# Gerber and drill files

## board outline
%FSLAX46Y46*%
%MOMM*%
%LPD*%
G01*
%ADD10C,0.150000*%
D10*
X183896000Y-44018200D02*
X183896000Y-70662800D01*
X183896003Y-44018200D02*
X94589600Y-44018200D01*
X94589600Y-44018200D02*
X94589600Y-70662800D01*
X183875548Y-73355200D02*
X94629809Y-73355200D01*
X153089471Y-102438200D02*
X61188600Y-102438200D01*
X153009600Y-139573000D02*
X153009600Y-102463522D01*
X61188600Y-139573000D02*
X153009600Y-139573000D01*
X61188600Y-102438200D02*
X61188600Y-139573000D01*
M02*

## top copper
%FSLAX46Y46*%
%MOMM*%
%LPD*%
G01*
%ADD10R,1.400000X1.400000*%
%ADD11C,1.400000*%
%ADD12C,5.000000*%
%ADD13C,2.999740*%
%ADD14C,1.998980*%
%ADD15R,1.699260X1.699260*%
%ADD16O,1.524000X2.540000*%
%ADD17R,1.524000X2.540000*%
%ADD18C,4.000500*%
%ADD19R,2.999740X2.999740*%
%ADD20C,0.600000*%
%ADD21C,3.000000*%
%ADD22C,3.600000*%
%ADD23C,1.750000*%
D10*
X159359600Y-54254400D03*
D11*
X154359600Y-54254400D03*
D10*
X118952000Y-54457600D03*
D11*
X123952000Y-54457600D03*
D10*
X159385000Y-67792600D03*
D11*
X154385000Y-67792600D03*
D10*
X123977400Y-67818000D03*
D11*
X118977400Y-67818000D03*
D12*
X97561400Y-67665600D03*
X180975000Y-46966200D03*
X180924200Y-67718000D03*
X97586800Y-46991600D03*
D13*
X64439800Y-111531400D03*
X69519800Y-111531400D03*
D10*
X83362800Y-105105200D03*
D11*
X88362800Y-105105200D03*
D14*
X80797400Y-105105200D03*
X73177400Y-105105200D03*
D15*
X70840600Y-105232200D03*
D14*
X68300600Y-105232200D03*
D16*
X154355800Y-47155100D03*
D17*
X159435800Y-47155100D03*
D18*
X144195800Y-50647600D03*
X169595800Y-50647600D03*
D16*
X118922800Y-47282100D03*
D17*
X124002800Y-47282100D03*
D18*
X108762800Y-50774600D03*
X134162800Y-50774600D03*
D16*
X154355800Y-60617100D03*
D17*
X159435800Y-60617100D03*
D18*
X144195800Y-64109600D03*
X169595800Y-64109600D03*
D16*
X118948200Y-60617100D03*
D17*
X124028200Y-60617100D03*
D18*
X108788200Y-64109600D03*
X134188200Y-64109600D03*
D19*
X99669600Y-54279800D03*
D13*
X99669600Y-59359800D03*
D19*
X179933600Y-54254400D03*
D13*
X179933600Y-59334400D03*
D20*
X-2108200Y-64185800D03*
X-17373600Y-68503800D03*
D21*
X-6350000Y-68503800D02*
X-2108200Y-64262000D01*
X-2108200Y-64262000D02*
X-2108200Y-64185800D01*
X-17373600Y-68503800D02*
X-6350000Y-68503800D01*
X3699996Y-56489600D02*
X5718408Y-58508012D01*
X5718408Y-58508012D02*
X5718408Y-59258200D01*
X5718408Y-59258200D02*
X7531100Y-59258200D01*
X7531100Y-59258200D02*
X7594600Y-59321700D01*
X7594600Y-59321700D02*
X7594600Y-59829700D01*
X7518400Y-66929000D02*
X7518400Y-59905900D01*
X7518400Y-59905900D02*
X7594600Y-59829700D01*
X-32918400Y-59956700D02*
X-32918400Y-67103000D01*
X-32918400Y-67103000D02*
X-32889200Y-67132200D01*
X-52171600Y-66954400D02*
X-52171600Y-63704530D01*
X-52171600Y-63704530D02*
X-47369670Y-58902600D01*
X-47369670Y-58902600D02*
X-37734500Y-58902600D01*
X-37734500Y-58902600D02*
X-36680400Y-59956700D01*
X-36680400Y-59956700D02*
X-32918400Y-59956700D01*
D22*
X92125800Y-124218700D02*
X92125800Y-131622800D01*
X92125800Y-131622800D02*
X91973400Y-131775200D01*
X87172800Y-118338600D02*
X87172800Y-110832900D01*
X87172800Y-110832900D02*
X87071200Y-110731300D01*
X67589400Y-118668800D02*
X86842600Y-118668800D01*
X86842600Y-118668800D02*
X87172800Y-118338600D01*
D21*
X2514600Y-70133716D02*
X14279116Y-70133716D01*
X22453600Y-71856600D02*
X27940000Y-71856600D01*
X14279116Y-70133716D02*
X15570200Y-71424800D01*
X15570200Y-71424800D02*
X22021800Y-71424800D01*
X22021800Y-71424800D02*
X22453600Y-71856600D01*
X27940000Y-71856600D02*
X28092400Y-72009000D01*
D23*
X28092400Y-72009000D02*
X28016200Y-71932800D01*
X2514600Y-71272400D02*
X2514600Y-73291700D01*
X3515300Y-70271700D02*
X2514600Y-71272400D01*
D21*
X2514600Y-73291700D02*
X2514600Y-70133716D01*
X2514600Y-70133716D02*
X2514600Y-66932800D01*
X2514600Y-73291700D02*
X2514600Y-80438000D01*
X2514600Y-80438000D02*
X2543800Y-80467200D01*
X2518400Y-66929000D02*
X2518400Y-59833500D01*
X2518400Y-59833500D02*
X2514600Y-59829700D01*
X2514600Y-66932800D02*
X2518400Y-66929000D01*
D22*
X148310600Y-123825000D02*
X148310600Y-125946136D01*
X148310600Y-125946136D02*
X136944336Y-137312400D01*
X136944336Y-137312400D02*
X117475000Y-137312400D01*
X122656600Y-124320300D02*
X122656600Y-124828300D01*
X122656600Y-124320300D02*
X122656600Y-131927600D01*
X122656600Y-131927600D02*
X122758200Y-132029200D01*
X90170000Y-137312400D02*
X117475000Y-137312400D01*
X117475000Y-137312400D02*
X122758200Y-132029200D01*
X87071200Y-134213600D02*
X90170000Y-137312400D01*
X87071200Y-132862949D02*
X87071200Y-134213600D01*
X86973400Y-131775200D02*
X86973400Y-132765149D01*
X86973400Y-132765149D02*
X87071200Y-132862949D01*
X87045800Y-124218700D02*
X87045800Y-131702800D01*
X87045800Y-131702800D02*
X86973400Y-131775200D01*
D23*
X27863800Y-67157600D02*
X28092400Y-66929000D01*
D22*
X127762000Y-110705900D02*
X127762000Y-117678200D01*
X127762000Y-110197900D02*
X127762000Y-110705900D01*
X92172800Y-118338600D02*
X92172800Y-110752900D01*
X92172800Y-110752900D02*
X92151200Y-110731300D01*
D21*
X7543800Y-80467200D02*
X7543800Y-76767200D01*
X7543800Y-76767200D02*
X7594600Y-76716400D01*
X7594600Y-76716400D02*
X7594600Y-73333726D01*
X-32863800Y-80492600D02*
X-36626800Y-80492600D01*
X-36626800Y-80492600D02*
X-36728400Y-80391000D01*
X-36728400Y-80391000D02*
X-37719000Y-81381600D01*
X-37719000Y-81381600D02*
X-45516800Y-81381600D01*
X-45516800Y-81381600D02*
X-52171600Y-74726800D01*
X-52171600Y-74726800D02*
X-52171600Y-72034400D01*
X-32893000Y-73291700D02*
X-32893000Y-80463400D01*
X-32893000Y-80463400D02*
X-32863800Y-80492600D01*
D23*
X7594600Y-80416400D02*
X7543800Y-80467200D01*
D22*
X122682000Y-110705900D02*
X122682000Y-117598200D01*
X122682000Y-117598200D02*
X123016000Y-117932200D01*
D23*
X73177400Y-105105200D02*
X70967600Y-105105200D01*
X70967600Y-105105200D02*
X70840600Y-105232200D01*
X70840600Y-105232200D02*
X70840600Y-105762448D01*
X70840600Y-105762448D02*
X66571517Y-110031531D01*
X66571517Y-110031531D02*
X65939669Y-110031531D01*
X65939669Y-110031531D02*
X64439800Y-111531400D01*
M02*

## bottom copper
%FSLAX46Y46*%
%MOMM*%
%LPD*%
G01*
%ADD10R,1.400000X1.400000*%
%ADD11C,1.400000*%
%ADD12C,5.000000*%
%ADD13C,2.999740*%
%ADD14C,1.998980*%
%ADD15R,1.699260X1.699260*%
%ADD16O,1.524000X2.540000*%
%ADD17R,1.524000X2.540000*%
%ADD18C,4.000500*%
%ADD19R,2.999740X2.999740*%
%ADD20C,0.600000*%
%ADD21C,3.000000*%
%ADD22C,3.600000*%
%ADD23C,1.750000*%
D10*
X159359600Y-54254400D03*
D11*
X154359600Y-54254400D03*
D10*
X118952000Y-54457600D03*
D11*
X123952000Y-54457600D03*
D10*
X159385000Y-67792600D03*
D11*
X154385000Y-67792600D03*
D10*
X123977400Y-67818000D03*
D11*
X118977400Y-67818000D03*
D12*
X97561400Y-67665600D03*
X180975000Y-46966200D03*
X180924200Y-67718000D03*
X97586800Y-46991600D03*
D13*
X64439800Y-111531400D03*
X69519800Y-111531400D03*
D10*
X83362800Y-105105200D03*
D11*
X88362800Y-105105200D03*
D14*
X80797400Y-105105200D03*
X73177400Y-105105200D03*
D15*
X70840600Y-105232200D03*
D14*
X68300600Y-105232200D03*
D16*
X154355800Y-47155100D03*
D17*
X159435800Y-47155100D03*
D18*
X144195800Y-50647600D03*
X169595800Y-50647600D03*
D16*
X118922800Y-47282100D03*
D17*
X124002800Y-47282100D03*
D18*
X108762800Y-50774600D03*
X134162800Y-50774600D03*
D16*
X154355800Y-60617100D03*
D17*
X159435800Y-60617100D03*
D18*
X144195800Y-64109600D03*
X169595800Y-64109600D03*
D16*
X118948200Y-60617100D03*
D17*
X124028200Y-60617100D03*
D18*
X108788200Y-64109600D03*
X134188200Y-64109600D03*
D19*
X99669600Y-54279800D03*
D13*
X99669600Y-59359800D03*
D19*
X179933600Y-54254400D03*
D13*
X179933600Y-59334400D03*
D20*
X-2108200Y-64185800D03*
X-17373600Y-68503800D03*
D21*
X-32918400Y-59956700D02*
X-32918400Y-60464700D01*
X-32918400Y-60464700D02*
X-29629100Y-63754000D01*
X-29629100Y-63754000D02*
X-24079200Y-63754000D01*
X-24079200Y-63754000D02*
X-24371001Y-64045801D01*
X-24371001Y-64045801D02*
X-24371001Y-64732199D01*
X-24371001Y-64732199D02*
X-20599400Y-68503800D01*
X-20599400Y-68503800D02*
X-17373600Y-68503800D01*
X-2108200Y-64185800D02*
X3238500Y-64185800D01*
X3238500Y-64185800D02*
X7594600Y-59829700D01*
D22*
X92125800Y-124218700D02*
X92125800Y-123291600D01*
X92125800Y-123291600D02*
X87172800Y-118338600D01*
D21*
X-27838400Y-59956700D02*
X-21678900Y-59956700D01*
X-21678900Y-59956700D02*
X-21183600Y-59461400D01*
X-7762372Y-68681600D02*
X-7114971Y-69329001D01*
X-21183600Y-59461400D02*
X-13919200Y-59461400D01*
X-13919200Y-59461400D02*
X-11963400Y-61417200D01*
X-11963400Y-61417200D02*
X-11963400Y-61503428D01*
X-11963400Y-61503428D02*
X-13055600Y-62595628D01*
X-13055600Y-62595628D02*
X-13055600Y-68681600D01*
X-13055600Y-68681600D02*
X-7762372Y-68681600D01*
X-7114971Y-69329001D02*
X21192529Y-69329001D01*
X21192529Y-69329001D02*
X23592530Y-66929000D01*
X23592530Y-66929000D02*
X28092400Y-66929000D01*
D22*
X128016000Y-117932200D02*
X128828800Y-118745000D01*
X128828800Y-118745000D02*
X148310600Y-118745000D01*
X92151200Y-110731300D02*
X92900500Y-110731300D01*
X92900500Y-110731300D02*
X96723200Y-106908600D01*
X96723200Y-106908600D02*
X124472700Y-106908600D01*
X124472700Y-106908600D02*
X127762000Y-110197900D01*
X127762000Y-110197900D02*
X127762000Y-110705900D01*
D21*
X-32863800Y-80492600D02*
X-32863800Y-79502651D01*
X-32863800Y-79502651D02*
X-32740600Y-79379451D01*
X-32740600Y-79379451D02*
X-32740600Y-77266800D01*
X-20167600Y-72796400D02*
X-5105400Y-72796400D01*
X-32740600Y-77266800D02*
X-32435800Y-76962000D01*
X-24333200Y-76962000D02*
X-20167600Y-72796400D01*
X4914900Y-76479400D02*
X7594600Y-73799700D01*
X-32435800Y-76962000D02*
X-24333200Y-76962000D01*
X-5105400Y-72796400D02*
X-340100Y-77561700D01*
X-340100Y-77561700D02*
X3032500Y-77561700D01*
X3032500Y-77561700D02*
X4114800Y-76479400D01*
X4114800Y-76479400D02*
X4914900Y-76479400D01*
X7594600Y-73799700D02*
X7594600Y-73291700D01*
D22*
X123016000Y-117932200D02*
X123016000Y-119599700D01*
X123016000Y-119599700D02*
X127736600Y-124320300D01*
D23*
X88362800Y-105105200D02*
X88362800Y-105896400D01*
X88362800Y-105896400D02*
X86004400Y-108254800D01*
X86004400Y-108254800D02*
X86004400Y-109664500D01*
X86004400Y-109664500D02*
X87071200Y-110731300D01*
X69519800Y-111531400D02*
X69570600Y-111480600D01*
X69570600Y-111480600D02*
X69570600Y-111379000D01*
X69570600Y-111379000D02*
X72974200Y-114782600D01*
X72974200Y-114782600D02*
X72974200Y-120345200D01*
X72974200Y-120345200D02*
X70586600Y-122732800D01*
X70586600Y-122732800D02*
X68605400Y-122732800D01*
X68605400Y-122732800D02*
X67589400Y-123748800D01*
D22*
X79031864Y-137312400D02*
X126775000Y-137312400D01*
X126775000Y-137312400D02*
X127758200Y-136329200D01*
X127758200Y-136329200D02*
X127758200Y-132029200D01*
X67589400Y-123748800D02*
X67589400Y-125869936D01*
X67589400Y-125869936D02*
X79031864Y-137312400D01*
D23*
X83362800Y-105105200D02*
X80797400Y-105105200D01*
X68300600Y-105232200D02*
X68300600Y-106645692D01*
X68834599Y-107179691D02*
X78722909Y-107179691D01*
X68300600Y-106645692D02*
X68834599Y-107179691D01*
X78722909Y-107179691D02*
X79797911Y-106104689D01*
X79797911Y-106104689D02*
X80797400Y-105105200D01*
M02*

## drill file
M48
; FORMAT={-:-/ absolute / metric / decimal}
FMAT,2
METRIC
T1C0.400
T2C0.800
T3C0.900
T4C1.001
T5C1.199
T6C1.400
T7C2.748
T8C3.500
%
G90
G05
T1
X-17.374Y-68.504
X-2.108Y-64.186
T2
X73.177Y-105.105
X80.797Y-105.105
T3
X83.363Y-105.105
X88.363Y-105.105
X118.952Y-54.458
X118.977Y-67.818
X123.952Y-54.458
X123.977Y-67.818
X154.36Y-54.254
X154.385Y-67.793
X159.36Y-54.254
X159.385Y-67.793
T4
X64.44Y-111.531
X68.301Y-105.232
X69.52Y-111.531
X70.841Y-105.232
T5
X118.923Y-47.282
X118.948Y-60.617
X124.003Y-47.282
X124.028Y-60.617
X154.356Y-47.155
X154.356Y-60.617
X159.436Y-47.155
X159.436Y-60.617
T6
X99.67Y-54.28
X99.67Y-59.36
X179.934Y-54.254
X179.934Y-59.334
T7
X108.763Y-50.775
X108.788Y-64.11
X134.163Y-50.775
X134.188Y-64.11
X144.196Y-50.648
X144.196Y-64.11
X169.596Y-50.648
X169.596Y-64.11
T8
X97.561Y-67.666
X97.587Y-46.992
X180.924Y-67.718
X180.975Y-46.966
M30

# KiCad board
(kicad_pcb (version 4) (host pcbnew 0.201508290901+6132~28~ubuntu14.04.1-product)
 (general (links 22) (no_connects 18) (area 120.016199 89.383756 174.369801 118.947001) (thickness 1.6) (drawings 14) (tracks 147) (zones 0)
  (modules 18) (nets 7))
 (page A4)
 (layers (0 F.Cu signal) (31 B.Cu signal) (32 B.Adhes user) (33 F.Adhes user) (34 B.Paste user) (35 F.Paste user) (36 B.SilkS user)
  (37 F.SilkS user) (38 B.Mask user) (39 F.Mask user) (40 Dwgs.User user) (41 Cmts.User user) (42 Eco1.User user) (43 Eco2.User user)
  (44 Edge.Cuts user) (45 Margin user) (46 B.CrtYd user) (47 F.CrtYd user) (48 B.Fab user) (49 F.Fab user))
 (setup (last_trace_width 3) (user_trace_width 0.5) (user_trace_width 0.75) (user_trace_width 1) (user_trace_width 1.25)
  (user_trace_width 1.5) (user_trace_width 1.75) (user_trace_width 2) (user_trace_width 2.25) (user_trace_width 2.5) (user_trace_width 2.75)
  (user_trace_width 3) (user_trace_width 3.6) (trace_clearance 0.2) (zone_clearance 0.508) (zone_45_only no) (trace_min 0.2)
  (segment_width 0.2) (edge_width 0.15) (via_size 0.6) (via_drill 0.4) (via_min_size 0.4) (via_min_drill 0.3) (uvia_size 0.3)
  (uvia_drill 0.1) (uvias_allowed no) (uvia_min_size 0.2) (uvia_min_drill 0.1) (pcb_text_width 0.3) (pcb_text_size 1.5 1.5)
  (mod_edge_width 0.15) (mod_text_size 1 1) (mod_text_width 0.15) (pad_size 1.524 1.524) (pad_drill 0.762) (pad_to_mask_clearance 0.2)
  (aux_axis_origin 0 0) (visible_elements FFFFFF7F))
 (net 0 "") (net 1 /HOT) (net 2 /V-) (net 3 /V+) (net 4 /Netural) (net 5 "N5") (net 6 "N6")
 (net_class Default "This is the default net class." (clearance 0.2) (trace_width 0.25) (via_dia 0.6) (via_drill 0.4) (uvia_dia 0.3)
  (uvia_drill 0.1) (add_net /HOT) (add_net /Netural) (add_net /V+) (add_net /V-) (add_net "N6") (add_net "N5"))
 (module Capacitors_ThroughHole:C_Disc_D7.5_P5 (layer F.Cu) (at 159.3596 54.2544 180)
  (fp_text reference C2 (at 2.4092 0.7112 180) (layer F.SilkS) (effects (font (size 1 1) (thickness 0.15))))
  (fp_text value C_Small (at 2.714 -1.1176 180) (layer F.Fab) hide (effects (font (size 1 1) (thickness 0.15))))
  (pad 1 thru_hole rect (at 0 0 180) (size 1.4 1.4) (drill 0.9) (layers *.Cu *.Mask F.SilkS) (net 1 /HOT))
  (pad 2 thru_hole circle (at 5 0 180) (size 1.4 1.4) (drill 0.9) (layers *.Cu *.Mask F.SilkS) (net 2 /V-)))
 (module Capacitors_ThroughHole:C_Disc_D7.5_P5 (layer F.Cu) (at 118.952 54.4576)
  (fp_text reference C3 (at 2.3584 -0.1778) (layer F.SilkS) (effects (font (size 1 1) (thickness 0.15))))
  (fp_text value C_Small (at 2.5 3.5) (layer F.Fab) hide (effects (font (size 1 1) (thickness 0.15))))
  (pad 1 thru_hole rect (at 0 0) (size 1.4 1.4) (drill 0.9) (layers *.Cu *.Mask F.SilkS) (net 1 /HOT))
  (pad 2 thru_hole circle (at 5 0) (size 1.4 1.4) (drill 0.9) (layers *.Cu *.Mask F.SilkS) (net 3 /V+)))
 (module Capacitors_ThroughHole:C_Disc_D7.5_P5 (layer F.Cu) (at 159.385 67.7926 180)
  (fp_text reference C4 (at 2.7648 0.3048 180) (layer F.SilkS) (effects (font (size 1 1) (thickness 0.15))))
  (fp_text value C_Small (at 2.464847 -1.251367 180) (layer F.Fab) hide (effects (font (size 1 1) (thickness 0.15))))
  (pad 1 thru_hole rect (at 0 0 180) (size 1.4 1.4) (drill 0.9) (layers *.Cu *.Mask F.SilkS) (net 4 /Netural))
  (pad 2 thru_hole circle (at 5 0 180) (size 1.4 1.4) (drill 0.9) (layers *.Cu *.Mask F.SilkS) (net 2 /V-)))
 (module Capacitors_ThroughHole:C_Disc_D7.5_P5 (layer F.Cu) (at 123.9774 67.818 180)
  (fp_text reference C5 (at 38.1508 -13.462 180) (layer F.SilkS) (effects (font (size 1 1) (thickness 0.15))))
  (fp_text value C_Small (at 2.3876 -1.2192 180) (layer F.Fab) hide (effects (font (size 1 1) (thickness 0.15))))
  (pad 1 thru_hole rect (at 0 0 180) (size 1.4 1.4) (drill 0.9) (layers *.Cu *.Mask F.SilkS) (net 3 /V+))
  (pad 2 thru_hole circle (at 5 0 180) (size 1.4 1.4) (drill 0.9) (layers *.Cu *.Mask F.SilkS) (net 4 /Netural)))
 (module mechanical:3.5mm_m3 (layer F.Cu) (at 97.5614 67.7656)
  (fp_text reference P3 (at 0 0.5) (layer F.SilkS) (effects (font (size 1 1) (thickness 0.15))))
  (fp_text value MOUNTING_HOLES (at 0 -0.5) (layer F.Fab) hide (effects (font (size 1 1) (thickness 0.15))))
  (pad 1 thru_hole circle (at 0 -0.1) (size 5 5) (drill 3.5) (layers *.Cu *.Mask F.SilkS)))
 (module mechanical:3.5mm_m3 (layer F.Cu) (at 180.975 47.0662)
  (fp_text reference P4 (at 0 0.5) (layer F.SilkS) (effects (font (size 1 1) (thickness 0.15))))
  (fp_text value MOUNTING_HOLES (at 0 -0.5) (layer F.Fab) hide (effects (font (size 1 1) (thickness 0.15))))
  (pad 1 thru_hole circle (at 0 -0.1) (size 5 5) (drill 3.5) (layers *.Cu *.Mask F.SilkS)))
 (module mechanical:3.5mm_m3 (layer F.Cu) (at 180.9242 67.818)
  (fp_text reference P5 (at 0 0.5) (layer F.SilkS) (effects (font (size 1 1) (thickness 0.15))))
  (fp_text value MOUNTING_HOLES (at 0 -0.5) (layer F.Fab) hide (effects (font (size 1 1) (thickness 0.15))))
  (pad 1 thru_hole circle (at 0 -0.1) (size 5 5) (drill 3.5) (layers *.Cu *.Mask F.SilkS)))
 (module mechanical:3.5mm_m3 (layer F.Cu) (at 97.5868 47.0916)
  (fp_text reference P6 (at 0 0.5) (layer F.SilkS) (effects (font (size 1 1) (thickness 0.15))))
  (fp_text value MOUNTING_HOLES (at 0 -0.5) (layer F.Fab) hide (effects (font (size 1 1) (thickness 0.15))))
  (pad 1 thru_hole circle (at 0 -0.1) (size 5 5) (drill 3.5) (layers *.Cu *.Mask F.SilkS)))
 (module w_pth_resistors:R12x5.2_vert (layer F.Cu) (at 64.4398 111.5314) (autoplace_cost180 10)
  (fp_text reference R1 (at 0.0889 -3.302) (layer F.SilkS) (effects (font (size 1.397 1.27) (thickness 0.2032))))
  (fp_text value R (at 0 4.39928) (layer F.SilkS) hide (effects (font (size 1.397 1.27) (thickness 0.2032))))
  (pad 1 thru_hole circle (at 0 0) (size 2.99974 2.99974) (drill 1.00076) (layers *.Cu *.Mask F.SilkS) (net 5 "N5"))
  (pad 2 thru_hole circle (at 5.08 0) (size 2.99974 2.99974) (drill 1.00076) (layers *.Cu *.Mask F.SilkS) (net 4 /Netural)))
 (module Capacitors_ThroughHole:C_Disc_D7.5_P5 (layer F.Cu) (at 83.3628 105.1052)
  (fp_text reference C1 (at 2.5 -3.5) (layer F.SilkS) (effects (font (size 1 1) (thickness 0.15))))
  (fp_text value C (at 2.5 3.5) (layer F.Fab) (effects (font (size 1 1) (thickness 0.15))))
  (pad 1 thru_hole rect (at 0 0) (size 1.4 1.4) (drill 0.9) (layers *.Cu *.Mask F.SilkS) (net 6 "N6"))
  (pad 2 thru_hole circle (at 5 0) (size 1.4 1.4) (drill 0.9) (layers *.Cu *.Mask F.SilkS) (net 1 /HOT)))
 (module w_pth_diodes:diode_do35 (layer F.Cu) (at 76.9874 105.1052 180)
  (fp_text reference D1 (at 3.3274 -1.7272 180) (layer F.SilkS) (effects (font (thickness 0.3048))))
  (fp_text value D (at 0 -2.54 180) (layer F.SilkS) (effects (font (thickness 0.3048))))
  (pad 1 thru_hole circle (at -3.81 0 180) (size 1.99898 1.99898) (drill 0.8001) (layers *.Cu *.Mask F.SilkS) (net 6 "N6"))
  (pad 2 thru_hole circle (at 3.81 0 180) (size 1.99898 1.99898) (drill 0.8001) (layers *.Cu *.Mask F.SilkS) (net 5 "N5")))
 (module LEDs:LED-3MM (layer F.Cu) (at 70.8406 105.2322 180)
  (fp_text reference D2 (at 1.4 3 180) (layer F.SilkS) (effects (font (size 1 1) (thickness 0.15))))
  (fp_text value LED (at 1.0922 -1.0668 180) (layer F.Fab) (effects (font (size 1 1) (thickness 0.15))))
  (pad 1 thru_hole rect (at 0 0 270) (size 1.69926 1.69926) (drill 1.00076) (layers *.Cu *.Mask F.SilkS) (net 5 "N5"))
  (pad 2 thru_hole circle (at 2.54 0 180) (size 1.99898 1.99898) (drill 1.00076) (layers *.Cu *.Mask F.SilkS) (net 6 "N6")))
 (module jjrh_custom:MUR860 (layer F.Cu) (at 156.8958 47.1551 180)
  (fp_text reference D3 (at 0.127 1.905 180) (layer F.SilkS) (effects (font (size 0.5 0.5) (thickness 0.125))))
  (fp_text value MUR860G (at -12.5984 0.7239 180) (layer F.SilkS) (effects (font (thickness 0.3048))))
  (pad 2 thru_hole oval (at 2.54 0 180) (size 1.524 2.54) (drill 1.19888) (layers *.Cu *.Mask F.SilkS) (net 2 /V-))
  (pad 1 thru_hole rect (at -2.54 0 180) (size 1.524 2.54) (drill oval 1.19888) (layers *.Cu *.Mask F.SilkS) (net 1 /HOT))
  (pad "" thru_hole circle (at 12.7 -3.4925 180) (size 4.0005 4.0005) (drill 2.74828) (layers *.Cu *.Mask F.SilkS))
  (pad "" thru_hole circle (at -12.7 -3.4925 180) (size 4.0005 4.0005) (drill 2.74828) (layers *.Cu *.Mask F.SilkS)))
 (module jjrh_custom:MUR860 (layer F.Cu) (at 121.4628 47.2821 180)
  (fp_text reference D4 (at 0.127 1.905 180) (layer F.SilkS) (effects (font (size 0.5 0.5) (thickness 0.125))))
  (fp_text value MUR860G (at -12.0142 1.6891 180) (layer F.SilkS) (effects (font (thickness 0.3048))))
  (pad 2 thru_hole oval (at 2.54 0 180) (size 1.524 2.54) (drill 1.19888) (layers *.Cu *.Mask F.SilkS) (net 1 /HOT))
  (pad 1 thru_hole rect (at -2.54 0 180) (size 1.524 2.54) (drill oval 1.19888) (layers *.Cu *.Mask F.SilkS) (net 3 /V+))
  (pad "" thru_hole circle (at 12.7 -3.4925 180) (size 4.0005 4.0005) (drill 2.74828) (layers *.Cu *.Mask F.SilkS))
  (pad "" thru_hole circle (at -12.7 -3.4925 180) (size 4.0005 4.0005) (drill 2.74828) (layers *.Cu *.Mask F.SilkS)))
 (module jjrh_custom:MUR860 (layer F.Cu) (at 156.8958 60.6171 180)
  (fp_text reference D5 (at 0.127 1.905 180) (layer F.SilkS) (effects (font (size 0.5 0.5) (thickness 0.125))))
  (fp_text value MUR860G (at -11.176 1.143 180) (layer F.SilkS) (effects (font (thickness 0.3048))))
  (pad 2 thru_hole oval (at 2.54 0 180) (size 1.524 2.54) (drill 1.19888) (layers *.Cu *.Mask F.SilkS) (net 2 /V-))
  (pad 1 thru_hole rect (at -2.54 0 180) (size 1.524 2.54) (drill oval 1.19888) (layers *.Cu *.Mask F.SilkS) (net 4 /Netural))
  (pad "" thru_hole circle (at 12.7 -3.4925 180) (size 4.0005 4.0005) (drill 2.74828) (layers *.Cu *.Mask F.SilkS))
  (pad "" thru_hole circle (at -12.7 -3.4925 180) (size 4.0005 4.0005) (drill 2.74828) (layers *.Cu *.Mask F.SilkS)))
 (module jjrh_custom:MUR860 (layer F.Cu) (at 121.4882 60.6171 180)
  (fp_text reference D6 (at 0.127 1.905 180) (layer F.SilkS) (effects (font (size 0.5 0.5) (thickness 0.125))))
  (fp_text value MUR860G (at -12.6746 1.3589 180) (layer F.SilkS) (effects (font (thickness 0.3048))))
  (pad 2 thru_hole oval (at 2.54 0 180) (size 1.524 2.54) (drill 1.19888) (layers *.Cu *.Mask F.SilkS) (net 4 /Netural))
  (pad 1 thru_hole rect (at -2.54 0 180) (size 1.524 2.54) (drill oval 1.19888) (layers *.Cu *.Mask F.SilkS) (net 3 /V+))
  (pad "" thru_hole circle (at 12.7 -3.4925 180) (size 4.0005 4.0005) (drill 2.74828) (layers *.Cu *.Mask F.SilkS))
  (pad "" thru_hole circle (at -12.7 -3.4925 180) (size 4.0005 4.0005) (drill 2.74828) (layers *.Cu *.Mask F.SilkS)))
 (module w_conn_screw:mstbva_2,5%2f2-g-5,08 (layer F.Cu) (at 99.6696 56.8198 270)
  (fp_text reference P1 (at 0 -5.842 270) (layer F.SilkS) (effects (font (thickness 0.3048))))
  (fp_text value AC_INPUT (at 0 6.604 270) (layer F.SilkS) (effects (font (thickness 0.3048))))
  (pad 1 thru_hole rect (at -2.54 0 270) (size 2.99974 2.99974) (drill 1.39954) (layers *.Cu *.Mask F.SilkS) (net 1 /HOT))
  (pad 2 thru_hole circle (at 2.54 0 270) (size 2.99974 2.99974) (drill 1.39954) (layers *.Cu *.Mask F.SilkS) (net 4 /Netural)))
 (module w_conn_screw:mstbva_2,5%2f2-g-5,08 (layer F.Cu) (at 179.9336 56.7944 270)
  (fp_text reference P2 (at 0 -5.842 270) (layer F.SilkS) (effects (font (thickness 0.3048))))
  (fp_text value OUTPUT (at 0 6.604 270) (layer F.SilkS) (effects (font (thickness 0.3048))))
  (pad 1 thru_hole rect (at -2.54 0 270) (size 2.99974 2.99974) (drill 1.39954) (layers *.Cu *.Mask F.SilkS) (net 3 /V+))
  (pad 2 thru_hole circle (at 2.54 0 270) (size 2.99974 2.99974) (drill 1.39954) (layers *.Cu *.Mask F.SilkS) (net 2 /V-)))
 (gr_line (start 183.896 44.0182) (end 183.896 70.6628) (layer Edge.Cuts) (width 0.15))
 (gr_line (start 183.896003 44.0182) (end 94.5896 44.0182) (layer Edge.Cuts) (width 0.15))
 (gr_line (start 94.5896 44.0182) (end 94.5896 70.6628) (layer Edge.Cuts) (width 0.15))
 (gr_line (start 183.875548 73.3552) (end 94.629809 73.3552) (layer Edge.Cuts) (width 0.15))
 (gr_line (start 153.089471 102.4382) (end 61.1886 102.4382) (layer Edge.Cuts) (width 0.15))
 (gr_line (start 153.0096 139.573) (end 153.0096 102.463522) (layer Edge.Cuts) (width 0.15))
 (gr_line (start 61.1886 139.573) (end 153.0096 139.573) (layer Edge.Cuts) (width 0.15))
 (gr_line (start 61.1886 102.4382) (end 61.1886 139.573) (layer Edge.Cuts) (width 0.15))
 (segment (start -32.9184 59.9567) (end -32.9184 60.4647) (width 3) (layer B.Cu) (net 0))
 (segment (start -32.9184 60.4647) (end -29.6291 63.754) (width 3) (layer B.Cu) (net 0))
 (segment (start -29.6291 63.754) (end -24.0792 63.754) (width 3) (layer B.Cu) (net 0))
 (segment (start -24.0792 63.754) (end -24.371001 64.045801) (width 3) (layer B.Cu) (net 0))
 (segment (start -24.371001 64.045801) (end -24.371001 64.732199) (width 3) (layer B.Cu) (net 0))
 (segment (start -24.371001 64.732199) (end -20.5994 68.5038) (width 3) (layer B.Cu) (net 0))
 (segment (start -20.5994 68.5038) (end -17.3736 68.5038) (width 3) (layer B.Cu) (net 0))
 (segment (start -2.1082 64.1858) (end 3.2385 64.1858) (width 3) (layer B.Cu) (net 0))
 (segment (start 3.2385 64.1858) (end 7.5946 59.8297) (width 3) (layer B.Cu) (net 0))
 (segment (start -6.35 68.5038) (end -2.1082 64.262) (width 3) (layer F.Cu) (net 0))
 (segment (start -2.1082 64.262) (end -2.1082 64.1858) (width 3) (layer F.Cu) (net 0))
 (via (at -2.1082 64.1858) (size 0.6) (drill 0.4) (layers F.Cu B.Cu) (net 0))
 (segment (start -17.3736 68.5038) (end -6.35 68.5038) (width 3) (layer F.Cu) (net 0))
 (via (at -17.3736 68.5038) (size 0.6) (drill 0.4) (layers F.Cu B.Cu) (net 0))
 (segment (start 3.699996 56.4896) (end 5.718408 58.508012) (width 3) (layer F.Cu) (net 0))
 (segment (start 5.718408 58.508012) (end 5.718408 59.2582) (width 3) (layer F.Cu) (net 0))
 (segment (start 5.718408 59.2582) (end 7.5311 59.2582) (width 3) (layer F.Cu) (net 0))
 (segment (start 7.5311 59.2582) (end 7.5946 59.3217) (width 3) (layer F.Cu) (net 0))
 (segment (start 7.5946 59.3217) (end 7.5946 59.8297) (width 3) (layer F.Cu) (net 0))
 (segment (start 7.5184 66.929) (end 7.5184 59.9059) (width 3) (layer F.Cu) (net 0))
 (segment (start 7.5184 59.9059) (end 7.5946 59.8297) (width 3) (layer F.Cu) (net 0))
 (segment (start -32.9184 59.9567) (end -32.9184 67.103) (width 3) (layer F.Cu) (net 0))
 (segment (start -32.9184 67.103) (end -32.8892 67.1322) (width 3) (layer F.Cu) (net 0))
 (segment (start -52.1716 66.9544) (end -52.1716 63.70453) (width 3) (layer F.Cu) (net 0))
 (segment (start -52.1716 63.70453) (end -47.36967 58.9026) (width 3) (layer F.Cu) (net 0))
 (segment (start -47.36967 58.9026) (end -37.7345 58.9026) (width 3) (layer F.Cu) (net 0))
 (segment (start -37.7345 58.9026) (end -36.6804 59.9567) (width 3) (layer F.Cu) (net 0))
 (segment (start -36.6804 59.9567) (end -32.9184 59.9567) (width 3) (layer F.Cu) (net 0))
 (segment (start 92.1258 124.2187) (end 92.1258 123.2916) (width 3.6) (layer B.Cu) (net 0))
 (segment (start 92.1258 123.2916) (end 87.1728 118.3386) (width 3.6) (layer B.Cu) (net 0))
 (segment (start 92.1258 124.2187) (end 92.1258 131.6228) (width 3.6) (layer F.Cu) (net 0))
 (segment (start 92.1258 131.6228) (end 91.9734 131.7752) (width 3.6) (layer F.Cu) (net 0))
 (segment (start 87.1728 118.3386) (end 87.1728 110.8329) (width 3.6) (layer F.Cu) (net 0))
 (segment (start 87.1728 110.8329) (end 87.0712 110.7313) (width 3.6) (layer F.Cu) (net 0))
 (segment (start 67.5894 118.6688) (end 86.8426 118.6688) (width 3.6) (layer F.Cu) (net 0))
 (segment (start 86.8426 118.6688) (end 87.1728 118.3386) (width 3.6) (layer F.Cu) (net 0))
 (segment (start 2.5146 70.133716) (end 14.279116 70.133716) (width 3) (layer F.Cu) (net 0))
 (segment (start 22.4536 71.8566) (end 27.94 71.8566) (width 3) (layer F.Cu) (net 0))
 (segment (start 14.279116 70.133716) (end 15.5702 71.4248) (width 3) (layer F.Cu) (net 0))
 (segment (start 15.5702 71.4248) (end 22.0218 71.4248) (width 3) (layer F.Cu) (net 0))
 (segment (start 22.0218 71.4248) (end 22.4536 71.8566) (width 3) (layer F.Cu) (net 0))
 (segment (start 27.94 71.8566) (end 28.0924 72.009) (width 3) (layer F.Cu) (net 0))
 (segment (start 28.0924 72.009) (end 28.0162 71.9328) (width 1.75) (layer F.Cu) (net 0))
 (segment (start 2.5146 71.2724) (end 2.5146 73.2917) (width 1.75) (layer F.Cu) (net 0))
 (segment (start 3.5153 70.2717) (end 2.5146 71.2724) (width 1.75) (layer F.Cu) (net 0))
 (segment (start 2.5146 73.2917) (end 2.5146 70.133716) (width 3) (layer F.Cu) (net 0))
 (segment (start 2.5146 70.133716) (end 2.5146 66.9328) (width 3) (layer F.Cu) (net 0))
 (segment (start 2.5146 73.2917) (end 2.5146 80.438) (width 3) (layer F.Cu) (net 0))
 (segment (start 2.5146 80.438) (end 2.5438 80.4672) (width 3) (layer F.Cu) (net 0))
 (segment (start 2.5184 66.929) (end 2.5184 59.8335) (width 3) (layer F.Cu) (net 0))
 (segment (start 2.5184 59.8335) (end 2.5146 59.8297) (width 3) (layer F.Cu) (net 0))
 (segment (start 2.5146 66.9328) (end 2.5184 66.929) (width 3) (layer F.Cu) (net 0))
 (segment (start 148.3106 123.825) (end 148.3106 125.946136) (width 3.6) (layer F.Cu) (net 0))
 (segment (start 148.3106 125.946136) (end 136.944336 137.3124) (width 3.6) (layer F.Cu) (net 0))
 (segment (start 136.944336 137.3124) (end 117.475 137.3124) (width 3.6) (layer F.Cu) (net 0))
 (segment (start 122.6566 124.3203) (end 122.6566 124.8283) (width 3.6) (layer F.Cu) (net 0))
 (segment (start 122.6566 124.3203) (end 122.6566 131.9276) (width 3.6) (layer F.Cu) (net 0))
 (segment (start 122.6566 131.9276) (end 122.7582 132.0292) (width 3.6) (layer F.Cu) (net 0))
 (segment (start 90.17 137.3124) (end 117.475 137.3124) (width 3.6) (layer F.Cu) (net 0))
 (segment (start 117.475 137.3124) (end 122.7582 132.0292) (width 3.6) (layer F.Cu) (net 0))
 (segment (start 87.0712 134.2136) (end 90.17 137.3124) (width 3.6) (layer F.Cu) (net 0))
 (segment (start 87.0712 132.862949) (end 87.0712 134.2136) (width 3.6) (layer F.Cu) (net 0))
 (segment (start 86.9734 131.7752) (end 86.9734 132.765149) (width 3.6) (layer F.Cu) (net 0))
 (segment (start 86.9734 132.765149) (end 87.0712 132.862949) (width 3.6) (layer F.Cu) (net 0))
 (segment (start 87.0458 124.2187) (end 87.0458 131.7028) (width 3.6) (layer F.Cu) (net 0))
 (segment (start 87.0458 131.7028) (end 86.9734 131.7752) (width 3.6) (layer F.Cu) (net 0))
 (segment (start -27.8384 59.9567) (end -21.6789 59.9567) (width 3) (layer B.Cu) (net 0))
 (segment (start -21.6789 59.9567) (end -21.1836 59.4614) (width 3) (layer B.Cu) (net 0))
 (segment (start -7.762372 68.6816) (end -7.114971 69.329001) (width 3) (layer B.Cu) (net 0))
 (segment (start -21.1836 59.4614) (end -13.9192 59.4614) (width 3) (layer B.Cu) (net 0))
 (segment (start -13.9192 59.4614) (end -11.9634 61.4172) (width 3) (layer B.Cu) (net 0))
 (segment (start -11.9634 61.4172) (end -11.9634 61.503428) (width 3) (layer B.Cu) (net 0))
 (segment (start -11.9634 61.503428) (end -13.0556 62.595628) (width 3) (layer B.Cu) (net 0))
 (segment (start -13.0556 62.595628) (end -13.0556 68.6816) (width 3) (layer B.Cu) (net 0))
 (segment (start -13.0556 68.6816) (end -7.762372 68.6816) (width 3) (layer B.Cu) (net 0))
 (segment (start -7.114971 69.329001) (end 21.192529 69.329001) (width 3) (layer B.Cu) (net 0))
 (segment (start 21.192529 69.329001) (end 23.59253 66.929) (width 3) (layer B.Cu) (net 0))
 (segment (start 23.59253 66.929) (end 28.0924 66.929) (width 3) (layer B.Cu) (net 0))
 (segment (start 27.8638 67.1576) (end 28.0924 66.929) (width 1.75) (layer F.Cu) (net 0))
 (segment (start 128.016 117.9322) (end 128.8288 118.745) (width 3.6) (layer B.Cu) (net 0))
 (segment (start 128.8288 118.745) (end 148.3106 118.745) (width 3.6) (layer B.Cu) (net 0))
 (segment (start 92.1512 110.7313) (end 92.9005 110.7313) (width 3.6) (layer B.Cu) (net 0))
 (segment (start 92.9005 110.7313) (end 96.7232 106.9086) (width 3.6) (layer B.Cu) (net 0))
 (segment (start 96.7232 106.9086) (end 124.4727 106.9086) (width 3.6) (layer B.Cu) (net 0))
 (segment (start 124.4727 106.9086) (end 127.762 110.1979) (width 3.6) (layer B.Cu) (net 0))
 (segment (start 127.762 110.1979) (end 127.762 110.7059) (width 3.6) (layer B.Cu) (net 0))
 (segment (start 127.762 110.7059) (end 127.762 117.6782) (width 3.6) (layer F.Cu) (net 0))
 (segment (start 127.762 110.1979) (end 127.762 110.7059) (width 3.6) (layer F.Cu) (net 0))
 (segment (start 92.1728 118.3386) (end 92.1728 110.7529) (width 3.6) (layer F.Cu) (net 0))
 (segment (start 92.1728 110.7529) (end 92.1512 110.7313) (width 3.6) (layer F.Cu) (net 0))
 (segment (start -32.8638 80.4926) (end -32.8638 79.502651) (width 3) (layer B.Cu) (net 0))
 (segment (start -32.8638 79.502651) (end -32.7406 79.379451) (width 3) (layer B.Cu) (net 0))
 (segment (start -32.7406 79.379451) (end -32.7406 77.2668) (width 3) (layer B.Cu) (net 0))
 (segment (start -20.1676 72.7964) (end -5.1054 72.7964) (width 3) (layer B.Cu) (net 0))
 (segment (start -32.7406 77.2668) (end -32.4358 76.962) (width 3) (layer B.Cu) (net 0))
 (segment (start -24.3332 76.962) (end -20.1676 72.7964) (width 3) (layer B.Cu) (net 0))
 (segment (start 4.9149 76.4794) (end 7.5946 73.7997) (width 3) (layer B.Cu) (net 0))
 (segment (start -32.4358 76.962) (end -24.3332 76.962) (width 3) (layer B.Cu) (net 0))
 (segment (start -5.1054 72.7964) (end -0.3401 77.5617) (width 3) (layer B.Cu) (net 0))
 (segment (start -0.3401 77.5617) (end 3.0325 77.5617) (width 3) (layer B.Cu) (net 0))
 (segment (start 3.0325 77.5617) (end 4.1148 76.4794) (width 3) (layer B.Cu) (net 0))
 (segment (start 4.1148 76.4794) (end 4.9149 76.4794) (width 3) (layer B.Cu) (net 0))
 (segment (start 7.5946 73.7997) (end 7.5946 73.2917) (width 3) (layer B.Cu) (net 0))
 (segment (start 7.5438 80.4672) (end 7.5438 76.7672) (width 3) (layer F.Cu) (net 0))
 (segment (start 7.5438 76.7672) (end 7.5946 76.7164) (width 3) (layer F.Cu) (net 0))
 (segment (start 7.5946 76.7164) (end 7.5946 73.333726) (width 3) (layer F.Cu) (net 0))
 (segment (start -32.8638 80.4926) (end -36.6268 80.4926) (width 3) (layer F.Cu) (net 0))
 (segment (start -36.6268 80.4926) (end -36.7284 80.391) (width 3) (layer F.Cu) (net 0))
 (segment (start -36.7284 80.391) (end -37.719 81.3816) (width 3) (layer F.Cu) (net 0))
 (segment (start -37.719 81.3816) (end -45.5168 81.3816) (width 3) (layer F.Cu) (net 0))
 (segment (start -45.5168 81.3816) (end -52.1716 74.7268) (width 3) (layer F.Cu) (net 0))
 (segment (start -52.1716 74.7268) (end -52.1716 72.0344) (width 3) (layer F.Cu) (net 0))
 (segment (start -32.893 73.2917) (end -32.893 80.4634) (width 3) (layer F.Cu) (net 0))
 (segment (start -32.893 80.4634) (end -32.8638 80.4926) (width 3) (layer F.Cu) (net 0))
 (segment (start 7.5946 80.4164) (end 7.5438 80.4672) (width 1.75) (layer F.Cu) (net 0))
 (segment (start 123.016 117.9322) (end 123.016 119.5997) (width 3.6) (layer B.Cu) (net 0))
 (segment (start 123.016 119.5997) (end 127.7366 124.3203) (width 3.6) (layer B.Cu) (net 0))
 (segment (start 122.682 110.7059) (end 122.682 117.5982) (width 3.6) (layer F.Cu) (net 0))
 (segment (start 122.682 117.5982) (end 123.016 117.9322) (width 3.6) (layer F.Cu) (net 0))
 (segment (start 88.3628 105.1052) (end 88.3628 105.8964) (width 1.75) (layer B.Cu) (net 1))
 (segment (start 88.3628 105.8964) (end 86.0044 108.2548) (width 1.75) (layer B.Cu) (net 1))
 (segment (start 86.0044 108.2548) (end 86.0044 109.6645) (width 1.75) (layer B.Cu) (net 1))
 (segment (start 86.0044 109.6645) (end 87.0712 110.7313) (width 1.75) (layer B.Cu) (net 1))
 (segment (start 69.5198 111.5314) (end 69.5706 111.4806) (width 1.75) (layer B.Cu) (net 4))
 (segment (start 69.5706 111.4806) (end 69.5706 111.379) (width 1.75) (layer B.Cu) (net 4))
 (segment (start 69.5706 111.379) (end 72.9742 114.7826) (width 1.75) (layer B.Cu) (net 4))
 (segment (start 72.9742 114.7826) (end 72.9742 120.3452) (width 1.75) (layer B.Cu) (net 4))
 (segment (start 72.9742 120.3452) (end 70.5866 122.7328) (width 1.75) (layer B.Cu) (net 4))
 (segment (start 70.5866 122.7328) (end 68.6054 122.7328) (width 1.75) (layer B.Cu) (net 4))
 (segment (start 68.6054 122.7328) (end 67.5894 123.7488) (width 1.75) (layer B.Cu) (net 4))
 (segment (start 79.031864 137.3124) (end 126.775 137.3124) (width 3.6) (layer B.Cu) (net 4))
 (segment (start 126.775 137.3124) (end 127.7582 136.3292) (width 3.6) (layer B.Cu) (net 4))
 (segment (start 127.7582 136.3292) (end 127.7582 132.0292) (width 3.6) (layer B.Cu) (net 4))
 (segment (start 67.5894 123.7488) (end 67.5894 125.869936) (width 3.6) (layer B.Cu) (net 4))
 (segment (start 67.5894 125.869936) (end 79.031864 137.3124) (width 3.6) (layer B.Cu) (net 4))
 (segment (start 83.3628 105.1052) (end 80.7974 105.1052) (width 1.75) (layer B.Cu) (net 6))
 (segment (start 68.3006 105.2322) (end 68.3006 106.645692) (width 1.75) (layer B.Cu) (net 6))
 (segment (start 68.834599 107.179691) (end 78.722909 107.179691) (width 1.75) (layer B.Cu) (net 6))
 (segment (start 68.3006 106.645692) (end 68.834599 107.179691) (width 1.75) (layer B.Cu) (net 6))
 (segment (start 78.722909 107.179691) (end 79.797911 106.104689) (width 1.75) (layer B.Cu) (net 6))
 (segment (start 79.797911 106.104689) (end 80.7974 105.1052) (width 1.75) (layer B.Cu) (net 6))
 (segment (start 73.1774 105.1052) (end 70.9676 105.1052) (width 1.75) (layer F.Cu) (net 5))
 (segment (start 70.9676 105.1052) (end 70.8406 105.2322) (width 1.75) (layer F.Cu) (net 5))
 (segment (start 70.8406 105.2322) (end 70.8406 105.762448) (width 1.75) (layer F.Cu) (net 5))
 (segment (start 70.8406 105.762448) (end 66.571517 110.031531) (width 1.75) (layer F.Cu) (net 5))
 (segment (start 66.571517 110.031531) (end 65.939669 110.031531) (width 1.75) (layer F.Cu) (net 5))
 (segment (start 65.939669 110.031531) (end 64.4398 111.5314) (width 1.75) (layer F.Cu) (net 5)))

